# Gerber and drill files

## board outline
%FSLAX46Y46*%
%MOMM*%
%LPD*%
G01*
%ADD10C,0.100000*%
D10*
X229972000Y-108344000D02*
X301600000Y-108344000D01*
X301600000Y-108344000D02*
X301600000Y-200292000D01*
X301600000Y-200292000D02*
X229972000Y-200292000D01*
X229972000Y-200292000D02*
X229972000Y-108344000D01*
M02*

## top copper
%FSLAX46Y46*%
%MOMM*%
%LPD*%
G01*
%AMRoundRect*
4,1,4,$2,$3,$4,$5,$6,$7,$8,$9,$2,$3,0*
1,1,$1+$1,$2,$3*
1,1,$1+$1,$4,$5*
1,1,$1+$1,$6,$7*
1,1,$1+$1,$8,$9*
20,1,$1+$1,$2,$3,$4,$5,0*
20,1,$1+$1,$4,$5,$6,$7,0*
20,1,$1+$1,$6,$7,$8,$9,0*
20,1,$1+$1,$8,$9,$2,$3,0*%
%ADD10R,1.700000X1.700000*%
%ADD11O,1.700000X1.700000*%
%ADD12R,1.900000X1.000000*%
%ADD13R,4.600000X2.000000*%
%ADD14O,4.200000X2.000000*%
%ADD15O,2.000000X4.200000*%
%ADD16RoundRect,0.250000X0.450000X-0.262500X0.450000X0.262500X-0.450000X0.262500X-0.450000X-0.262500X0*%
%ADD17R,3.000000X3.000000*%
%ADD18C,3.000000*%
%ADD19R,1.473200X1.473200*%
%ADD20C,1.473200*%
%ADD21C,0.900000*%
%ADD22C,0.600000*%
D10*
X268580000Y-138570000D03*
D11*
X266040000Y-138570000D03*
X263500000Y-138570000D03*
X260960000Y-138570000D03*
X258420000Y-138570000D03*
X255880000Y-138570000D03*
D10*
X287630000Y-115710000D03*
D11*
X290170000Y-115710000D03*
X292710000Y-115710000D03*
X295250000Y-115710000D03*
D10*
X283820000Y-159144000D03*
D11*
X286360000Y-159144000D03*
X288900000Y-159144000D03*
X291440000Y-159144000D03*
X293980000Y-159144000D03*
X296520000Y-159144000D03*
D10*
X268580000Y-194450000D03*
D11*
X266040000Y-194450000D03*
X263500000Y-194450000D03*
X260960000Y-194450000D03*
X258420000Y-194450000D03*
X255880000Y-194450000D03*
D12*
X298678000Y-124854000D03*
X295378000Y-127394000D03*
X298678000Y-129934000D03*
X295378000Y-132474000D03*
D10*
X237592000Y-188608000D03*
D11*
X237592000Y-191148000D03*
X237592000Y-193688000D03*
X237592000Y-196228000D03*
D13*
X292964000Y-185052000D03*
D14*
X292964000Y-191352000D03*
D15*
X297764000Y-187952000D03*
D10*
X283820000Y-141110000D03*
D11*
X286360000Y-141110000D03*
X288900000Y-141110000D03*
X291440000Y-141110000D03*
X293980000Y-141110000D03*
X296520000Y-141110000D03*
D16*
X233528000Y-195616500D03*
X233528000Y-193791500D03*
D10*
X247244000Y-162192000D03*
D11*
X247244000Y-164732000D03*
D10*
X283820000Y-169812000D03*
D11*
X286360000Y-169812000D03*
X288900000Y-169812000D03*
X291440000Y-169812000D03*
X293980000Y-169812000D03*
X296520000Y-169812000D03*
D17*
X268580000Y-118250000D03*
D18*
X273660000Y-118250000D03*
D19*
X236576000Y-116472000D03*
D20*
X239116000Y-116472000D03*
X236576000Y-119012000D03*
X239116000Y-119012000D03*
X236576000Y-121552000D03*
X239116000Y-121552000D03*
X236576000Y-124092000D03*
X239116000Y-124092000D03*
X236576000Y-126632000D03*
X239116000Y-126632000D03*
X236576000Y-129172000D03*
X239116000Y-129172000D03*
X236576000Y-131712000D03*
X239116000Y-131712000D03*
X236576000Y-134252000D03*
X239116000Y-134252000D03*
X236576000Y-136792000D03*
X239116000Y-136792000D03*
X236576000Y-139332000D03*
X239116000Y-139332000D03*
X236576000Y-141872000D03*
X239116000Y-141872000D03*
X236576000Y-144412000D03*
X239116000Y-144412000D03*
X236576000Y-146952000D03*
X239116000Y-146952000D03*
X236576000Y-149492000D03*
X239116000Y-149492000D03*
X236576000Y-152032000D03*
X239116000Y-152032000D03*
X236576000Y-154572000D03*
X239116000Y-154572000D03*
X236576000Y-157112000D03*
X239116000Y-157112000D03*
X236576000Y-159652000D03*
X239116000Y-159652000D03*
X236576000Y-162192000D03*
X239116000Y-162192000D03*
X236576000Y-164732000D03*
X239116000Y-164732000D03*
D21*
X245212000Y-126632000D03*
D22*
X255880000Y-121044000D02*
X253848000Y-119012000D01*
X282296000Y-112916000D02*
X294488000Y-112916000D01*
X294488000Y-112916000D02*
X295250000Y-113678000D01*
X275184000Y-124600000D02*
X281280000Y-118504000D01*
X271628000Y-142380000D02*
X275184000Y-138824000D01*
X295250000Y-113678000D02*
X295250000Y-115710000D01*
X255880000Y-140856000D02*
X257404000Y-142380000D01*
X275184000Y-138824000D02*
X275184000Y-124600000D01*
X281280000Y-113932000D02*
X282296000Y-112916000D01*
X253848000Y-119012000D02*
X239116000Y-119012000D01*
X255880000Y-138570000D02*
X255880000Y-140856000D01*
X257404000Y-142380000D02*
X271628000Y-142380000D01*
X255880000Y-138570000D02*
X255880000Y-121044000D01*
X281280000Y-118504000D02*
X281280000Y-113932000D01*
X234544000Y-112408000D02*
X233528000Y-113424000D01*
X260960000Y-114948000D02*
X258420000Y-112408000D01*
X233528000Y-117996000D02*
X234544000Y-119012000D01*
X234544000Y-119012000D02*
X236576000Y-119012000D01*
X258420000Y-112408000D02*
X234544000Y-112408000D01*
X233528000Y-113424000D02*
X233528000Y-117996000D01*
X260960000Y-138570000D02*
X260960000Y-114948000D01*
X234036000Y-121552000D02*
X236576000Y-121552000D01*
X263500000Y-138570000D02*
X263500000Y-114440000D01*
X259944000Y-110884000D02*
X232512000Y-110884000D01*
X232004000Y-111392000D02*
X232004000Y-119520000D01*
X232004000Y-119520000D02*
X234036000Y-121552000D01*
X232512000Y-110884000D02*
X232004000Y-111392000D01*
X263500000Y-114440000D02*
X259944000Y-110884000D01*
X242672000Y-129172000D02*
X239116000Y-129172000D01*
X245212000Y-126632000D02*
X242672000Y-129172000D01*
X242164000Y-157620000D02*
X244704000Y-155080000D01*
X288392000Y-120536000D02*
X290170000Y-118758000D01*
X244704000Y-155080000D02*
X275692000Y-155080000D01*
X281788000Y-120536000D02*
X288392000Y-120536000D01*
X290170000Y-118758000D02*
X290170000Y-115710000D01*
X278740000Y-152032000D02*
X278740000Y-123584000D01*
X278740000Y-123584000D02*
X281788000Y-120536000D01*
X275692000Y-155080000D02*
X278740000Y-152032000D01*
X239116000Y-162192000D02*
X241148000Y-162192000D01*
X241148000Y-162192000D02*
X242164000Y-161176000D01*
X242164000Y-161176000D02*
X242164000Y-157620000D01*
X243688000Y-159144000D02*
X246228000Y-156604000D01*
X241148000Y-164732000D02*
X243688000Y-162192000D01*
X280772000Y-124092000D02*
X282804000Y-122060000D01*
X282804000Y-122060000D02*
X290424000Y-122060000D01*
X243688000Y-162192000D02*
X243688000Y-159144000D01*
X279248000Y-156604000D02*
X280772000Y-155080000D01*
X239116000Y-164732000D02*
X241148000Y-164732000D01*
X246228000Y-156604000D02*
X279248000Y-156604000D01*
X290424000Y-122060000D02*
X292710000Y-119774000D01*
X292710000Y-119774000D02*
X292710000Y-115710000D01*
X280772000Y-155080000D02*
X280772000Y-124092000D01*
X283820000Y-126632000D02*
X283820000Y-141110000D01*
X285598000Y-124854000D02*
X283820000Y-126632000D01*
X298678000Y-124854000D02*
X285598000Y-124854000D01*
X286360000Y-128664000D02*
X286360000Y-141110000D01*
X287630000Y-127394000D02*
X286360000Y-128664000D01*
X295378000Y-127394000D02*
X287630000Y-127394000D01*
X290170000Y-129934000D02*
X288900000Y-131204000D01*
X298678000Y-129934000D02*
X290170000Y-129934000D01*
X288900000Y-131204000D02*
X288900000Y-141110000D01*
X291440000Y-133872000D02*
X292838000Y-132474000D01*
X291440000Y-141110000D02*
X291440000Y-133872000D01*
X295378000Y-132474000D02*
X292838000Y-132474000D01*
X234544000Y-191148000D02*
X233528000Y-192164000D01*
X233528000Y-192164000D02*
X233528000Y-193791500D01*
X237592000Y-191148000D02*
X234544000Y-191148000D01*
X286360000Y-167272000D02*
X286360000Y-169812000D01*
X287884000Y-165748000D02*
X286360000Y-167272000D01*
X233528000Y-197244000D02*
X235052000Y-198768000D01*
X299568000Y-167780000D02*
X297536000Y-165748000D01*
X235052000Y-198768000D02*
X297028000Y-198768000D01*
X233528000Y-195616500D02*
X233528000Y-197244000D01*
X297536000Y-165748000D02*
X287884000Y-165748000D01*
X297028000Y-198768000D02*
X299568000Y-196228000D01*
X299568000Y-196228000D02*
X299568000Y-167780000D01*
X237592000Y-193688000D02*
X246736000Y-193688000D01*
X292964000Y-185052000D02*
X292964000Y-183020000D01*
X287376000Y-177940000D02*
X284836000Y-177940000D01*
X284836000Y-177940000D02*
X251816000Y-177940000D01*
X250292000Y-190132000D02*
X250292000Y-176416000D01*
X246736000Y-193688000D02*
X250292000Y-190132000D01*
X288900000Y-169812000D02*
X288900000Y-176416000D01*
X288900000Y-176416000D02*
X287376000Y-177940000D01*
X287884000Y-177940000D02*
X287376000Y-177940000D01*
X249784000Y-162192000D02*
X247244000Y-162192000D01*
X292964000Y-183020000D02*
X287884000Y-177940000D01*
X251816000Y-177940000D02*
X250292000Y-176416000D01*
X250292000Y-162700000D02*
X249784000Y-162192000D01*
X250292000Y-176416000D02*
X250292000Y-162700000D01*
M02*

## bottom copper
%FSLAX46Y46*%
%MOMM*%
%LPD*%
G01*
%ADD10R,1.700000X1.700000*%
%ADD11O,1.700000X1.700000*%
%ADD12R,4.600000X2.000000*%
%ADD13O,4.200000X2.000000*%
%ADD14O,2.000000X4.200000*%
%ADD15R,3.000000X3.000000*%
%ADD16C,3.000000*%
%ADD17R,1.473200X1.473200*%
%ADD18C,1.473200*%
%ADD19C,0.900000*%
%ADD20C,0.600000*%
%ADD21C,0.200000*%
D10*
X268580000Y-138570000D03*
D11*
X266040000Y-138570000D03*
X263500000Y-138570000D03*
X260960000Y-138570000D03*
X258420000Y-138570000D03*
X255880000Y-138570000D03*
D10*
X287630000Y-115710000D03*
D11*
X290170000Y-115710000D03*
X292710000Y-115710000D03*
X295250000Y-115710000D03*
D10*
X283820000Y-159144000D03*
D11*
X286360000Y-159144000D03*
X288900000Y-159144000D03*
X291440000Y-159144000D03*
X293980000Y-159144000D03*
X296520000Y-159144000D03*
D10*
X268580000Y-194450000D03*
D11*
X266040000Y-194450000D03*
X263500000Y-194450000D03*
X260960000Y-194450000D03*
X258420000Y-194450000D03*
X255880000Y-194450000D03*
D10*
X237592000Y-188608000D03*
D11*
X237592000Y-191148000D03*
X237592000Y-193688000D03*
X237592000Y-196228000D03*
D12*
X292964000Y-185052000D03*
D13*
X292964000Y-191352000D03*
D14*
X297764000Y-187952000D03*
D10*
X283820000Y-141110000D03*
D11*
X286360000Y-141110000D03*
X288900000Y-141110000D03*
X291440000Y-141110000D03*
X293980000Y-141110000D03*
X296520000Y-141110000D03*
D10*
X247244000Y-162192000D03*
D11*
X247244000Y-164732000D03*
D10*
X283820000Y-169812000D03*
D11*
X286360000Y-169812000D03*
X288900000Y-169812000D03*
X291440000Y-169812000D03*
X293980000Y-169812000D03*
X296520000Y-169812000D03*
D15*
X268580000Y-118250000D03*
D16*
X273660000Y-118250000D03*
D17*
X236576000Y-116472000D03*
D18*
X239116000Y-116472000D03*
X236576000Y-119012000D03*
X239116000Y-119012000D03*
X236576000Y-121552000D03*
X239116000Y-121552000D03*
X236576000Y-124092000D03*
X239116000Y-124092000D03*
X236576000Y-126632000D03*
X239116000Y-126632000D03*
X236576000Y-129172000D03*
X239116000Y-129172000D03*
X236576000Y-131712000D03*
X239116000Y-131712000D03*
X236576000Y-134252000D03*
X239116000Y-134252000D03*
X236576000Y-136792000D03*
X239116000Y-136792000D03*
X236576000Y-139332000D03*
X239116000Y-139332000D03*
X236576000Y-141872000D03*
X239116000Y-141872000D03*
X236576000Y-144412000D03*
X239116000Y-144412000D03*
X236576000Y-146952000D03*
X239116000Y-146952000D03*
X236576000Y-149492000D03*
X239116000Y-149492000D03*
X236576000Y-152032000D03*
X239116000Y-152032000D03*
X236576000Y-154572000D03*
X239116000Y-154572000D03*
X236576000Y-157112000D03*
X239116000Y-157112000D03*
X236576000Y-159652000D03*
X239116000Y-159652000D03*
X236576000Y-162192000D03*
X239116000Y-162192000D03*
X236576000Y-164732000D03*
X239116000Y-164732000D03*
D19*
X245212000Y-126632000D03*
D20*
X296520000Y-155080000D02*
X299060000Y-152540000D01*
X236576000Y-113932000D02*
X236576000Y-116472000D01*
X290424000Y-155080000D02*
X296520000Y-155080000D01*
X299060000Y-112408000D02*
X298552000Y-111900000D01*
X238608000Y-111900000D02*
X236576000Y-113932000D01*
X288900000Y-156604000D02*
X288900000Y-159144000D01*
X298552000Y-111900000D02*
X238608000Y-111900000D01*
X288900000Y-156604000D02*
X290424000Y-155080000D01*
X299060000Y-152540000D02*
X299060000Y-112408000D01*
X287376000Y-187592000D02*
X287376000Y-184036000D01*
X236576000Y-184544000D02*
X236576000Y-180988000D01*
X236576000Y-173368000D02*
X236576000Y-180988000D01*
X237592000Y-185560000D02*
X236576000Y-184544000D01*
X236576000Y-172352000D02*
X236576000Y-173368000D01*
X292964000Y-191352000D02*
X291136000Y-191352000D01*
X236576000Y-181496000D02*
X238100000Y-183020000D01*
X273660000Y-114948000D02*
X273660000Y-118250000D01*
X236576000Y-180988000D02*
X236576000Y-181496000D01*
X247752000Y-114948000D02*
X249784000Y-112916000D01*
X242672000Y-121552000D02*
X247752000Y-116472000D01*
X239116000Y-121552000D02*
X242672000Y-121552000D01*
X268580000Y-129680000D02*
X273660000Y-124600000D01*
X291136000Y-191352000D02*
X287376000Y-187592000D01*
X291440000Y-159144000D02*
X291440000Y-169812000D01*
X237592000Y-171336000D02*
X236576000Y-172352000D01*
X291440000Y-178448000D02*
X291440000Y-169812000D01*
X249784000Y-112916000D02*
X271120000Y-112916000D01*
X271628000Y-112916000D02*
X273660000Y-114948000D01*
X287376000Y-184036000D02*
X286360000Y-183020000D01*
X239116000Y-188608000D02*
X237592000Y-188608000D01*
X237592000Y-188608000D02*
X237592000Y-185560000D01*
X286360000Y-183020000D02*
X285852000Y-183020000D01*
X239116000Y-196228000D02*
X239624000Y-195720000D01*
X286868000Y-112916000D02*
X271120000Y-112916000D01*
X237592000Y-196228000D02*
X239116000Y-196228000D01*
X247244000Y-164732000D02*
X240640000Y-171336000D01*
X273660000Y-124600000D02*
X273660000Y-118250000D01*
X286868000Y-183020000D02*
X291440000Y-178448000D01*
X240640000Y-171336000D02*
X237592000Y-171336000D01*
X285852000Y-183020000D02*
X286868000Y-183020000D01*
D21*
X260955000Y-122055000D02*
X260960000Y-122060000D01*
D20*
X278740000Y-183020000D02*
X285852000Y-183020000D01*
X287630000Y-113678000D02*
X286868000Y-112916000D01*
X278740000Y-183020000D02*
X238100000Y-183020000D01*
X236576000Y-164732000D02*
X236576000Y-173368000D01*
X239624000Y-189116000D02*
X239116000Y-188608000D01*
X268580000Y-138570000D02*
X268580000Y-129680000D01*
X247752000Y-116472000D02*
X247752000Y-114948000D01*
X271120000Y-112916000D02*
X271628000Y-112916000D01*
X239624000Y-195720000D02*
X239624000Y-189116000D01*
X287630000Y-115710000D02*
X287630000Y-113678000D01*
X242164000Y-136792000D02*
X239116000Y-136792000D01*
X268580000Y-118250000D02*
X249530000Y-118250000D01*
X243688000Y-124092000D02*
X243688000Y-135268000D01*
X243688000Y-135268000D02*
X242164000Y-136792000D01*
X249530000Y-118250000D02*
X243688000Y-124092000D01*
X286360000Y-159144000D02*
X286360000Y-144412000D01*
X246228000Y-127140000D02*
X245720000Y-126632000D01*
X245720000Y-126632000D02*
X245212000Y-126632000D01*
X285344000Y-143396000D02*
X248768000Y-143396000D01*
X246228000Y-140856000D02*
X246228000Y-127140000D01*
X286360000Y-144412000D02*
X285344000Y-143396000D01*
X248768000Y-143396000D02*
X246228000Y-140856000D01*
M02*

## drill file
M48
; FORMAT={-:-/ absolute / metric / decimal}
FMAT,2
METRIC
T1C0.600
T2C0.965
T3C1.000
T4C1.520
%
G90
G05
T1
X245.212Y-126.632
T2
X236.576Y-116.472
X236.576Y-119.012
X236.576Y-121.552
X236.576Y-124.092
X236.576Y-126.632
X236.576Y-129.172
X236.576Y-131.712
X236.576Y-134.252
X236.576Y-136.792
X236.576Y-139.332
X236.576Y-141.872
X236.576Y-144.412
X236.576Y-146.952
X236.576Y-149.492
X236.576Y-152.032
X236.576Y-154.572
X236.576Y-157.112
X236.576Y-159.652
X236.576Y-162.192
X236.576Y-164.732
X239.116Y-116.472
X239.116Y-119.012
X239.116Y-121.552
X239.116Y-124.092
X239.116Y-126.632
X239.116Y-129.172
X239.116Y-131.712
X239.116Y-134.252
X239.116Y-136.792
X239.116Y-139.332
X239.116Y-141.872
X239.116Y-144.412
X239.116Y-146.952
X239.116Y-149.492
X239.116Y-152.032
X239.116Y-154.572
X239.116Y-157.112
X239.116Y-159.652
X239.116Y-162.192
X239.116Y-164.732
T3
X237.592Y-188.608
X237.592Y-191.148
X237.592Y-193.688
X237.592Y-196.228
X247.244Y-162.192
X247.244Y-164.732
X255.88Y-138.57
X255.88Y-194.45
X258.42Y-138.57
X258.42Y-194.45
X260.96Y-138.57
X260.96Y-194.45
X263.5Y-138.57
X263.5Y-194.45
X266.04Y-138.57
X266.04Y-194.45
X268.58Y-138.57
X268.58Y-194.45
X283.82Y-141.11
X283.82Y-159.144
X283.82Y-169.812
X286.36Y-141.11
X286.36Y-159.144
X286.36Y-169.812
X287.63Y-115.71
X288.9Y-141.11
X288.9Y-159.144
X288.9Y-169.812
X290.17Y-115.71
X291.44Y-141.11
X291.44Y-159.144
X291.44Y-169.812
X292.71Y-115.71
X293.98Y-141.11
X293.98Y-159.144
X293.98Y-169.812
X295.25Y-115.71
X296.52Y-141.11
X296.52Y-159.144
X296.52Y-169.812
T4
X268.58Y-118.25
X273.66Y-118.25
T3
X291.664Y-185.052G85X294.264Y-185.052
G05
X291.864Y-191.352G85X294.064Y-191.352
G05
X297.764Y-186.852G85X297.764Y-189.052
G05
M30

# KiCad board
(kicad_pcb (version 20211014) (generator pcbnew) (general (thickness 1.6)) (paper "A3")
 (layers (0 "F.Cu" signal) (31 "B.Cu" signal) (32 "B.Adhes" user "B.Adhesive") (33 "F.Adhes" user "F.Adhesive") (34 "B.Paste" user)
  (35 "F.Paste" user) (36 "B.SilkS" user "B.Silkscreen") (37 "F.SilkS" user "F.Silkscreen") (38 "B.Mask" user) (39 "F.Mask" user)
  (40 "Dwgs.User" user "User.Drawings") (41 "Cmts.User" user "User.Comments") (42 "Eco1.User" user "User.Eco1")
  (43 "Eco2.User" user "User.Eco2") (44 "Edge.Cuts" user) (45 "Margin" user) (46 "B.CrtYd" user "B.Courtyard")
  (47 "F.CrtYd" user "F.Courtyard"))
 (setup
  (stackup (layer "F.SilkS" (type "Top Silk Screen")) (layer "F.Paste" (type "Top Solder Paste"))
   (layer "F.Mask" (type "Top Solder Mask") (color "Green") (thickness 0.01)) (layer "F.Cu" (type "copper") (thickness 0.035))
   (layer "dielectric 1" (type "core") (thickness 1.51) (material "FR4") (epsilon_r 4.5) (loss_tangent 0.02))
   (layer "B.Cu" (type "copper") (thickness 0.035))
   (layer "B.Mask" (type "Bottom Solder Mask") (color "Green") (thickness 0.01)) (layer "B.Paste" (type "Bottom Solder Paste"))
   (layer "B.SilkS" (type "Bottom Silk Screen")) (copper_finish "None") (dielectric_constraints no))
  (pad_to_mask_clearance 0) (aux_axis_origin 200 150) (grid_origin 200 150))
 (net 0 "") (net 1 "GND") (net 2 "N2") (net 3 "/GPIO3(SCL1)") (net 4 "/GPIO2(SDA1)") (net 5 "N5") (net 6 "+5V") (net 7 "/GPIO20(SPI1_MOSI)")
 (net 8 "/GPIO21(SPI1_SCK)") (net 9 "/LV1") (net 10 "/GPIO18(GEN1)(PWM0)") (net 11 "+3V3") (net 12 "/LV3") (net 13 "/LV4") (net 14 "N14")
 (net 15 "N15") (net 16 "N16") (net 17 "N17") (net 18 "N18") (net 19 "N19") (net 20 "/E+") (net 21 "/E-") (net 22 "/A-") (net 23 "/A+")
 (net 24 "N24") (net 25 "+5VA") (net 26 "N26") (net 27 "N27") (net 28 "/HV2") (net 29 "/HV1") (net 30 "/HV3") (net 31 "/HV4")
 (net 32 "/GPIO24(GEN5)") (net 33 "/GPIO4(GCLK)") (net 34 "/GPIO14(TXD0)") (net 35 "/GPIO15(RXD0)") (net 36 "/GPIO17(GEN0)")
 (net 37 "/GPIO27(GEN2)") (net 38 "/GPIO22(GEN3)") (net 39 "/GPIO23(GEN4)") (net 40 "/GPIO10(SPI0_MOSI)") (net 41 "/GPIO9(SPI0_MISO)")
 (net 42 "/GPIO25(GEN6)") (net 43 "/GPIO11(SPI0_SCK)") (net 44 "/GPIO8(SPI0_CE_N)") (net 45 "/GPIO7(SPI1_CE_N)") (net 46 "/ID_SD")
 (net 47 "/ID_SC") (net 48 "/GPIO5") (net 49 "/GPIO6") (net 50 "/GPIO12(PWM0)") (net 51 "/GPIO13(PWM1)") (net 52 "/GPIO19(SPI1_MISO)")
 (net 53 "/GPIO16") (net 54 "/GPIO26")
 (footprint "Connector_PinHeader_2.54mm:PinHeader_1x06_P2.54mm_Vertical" (layer "F.Cu") (at 268.58 138.57 -90)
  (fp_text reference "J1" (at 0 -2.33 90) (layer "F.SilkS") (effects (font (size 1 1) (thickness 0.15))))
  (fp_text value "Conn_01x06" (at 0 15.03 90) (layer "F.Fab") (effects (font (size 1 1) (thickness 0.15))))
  (pad "1" thru_hole rect (at 0 0 270) (size 1.7 1.7) (drill 1) (layers *.Cu *.Mask) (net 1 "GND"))
  (pad "2" thru_hole oval (at 0 2.54 270) (size 1.7 1.7) (drill 1) (layers *.Cu *.Mask) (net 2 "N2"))
  (pad "3" thru_hole oval (at 0 5.08 270) (size 1.7 1.7) (drill 1) (layers *.Cu *.Mask) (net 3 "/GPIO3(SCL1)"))
  (pad "4" thru_hole oval (at 0 7.62 270) (size 1.7 1.7) (drill 1) (layers *.Cu *.Mask) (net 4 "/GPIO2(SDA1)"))
  (pad "5" thru_hole oval (at 0 10.16 270) (size 1.7 1.7) (drill 1) (layers *.Cu *.Mask) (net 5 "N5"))
  (pad "6" thru_hole oval (at 0 12.7 270) (size 1.7 1.7) (drill 1) (layers *.Cu *.Mask) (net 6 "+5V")))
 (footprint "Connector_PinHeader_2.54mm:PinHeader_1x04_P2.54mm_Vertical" (layer "F.Cu") (at 287.63 115.71 90)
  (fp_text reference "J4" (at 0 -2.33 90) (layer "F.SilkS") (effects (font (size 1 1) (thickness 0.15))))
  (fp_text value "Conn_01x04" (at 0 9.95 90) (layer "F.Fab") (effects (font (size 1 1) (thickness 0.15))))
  (pad "1" thru_hole rect (at 0 0 90) (size 1.7 1.7) (drill 1) (layers *.Cu *.Mask) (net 1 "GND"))
  (pad "2" thru_hole oval (at 0 2.54 90) (size 1.7 1.7) (drill 1) (layers *.Cu *.Mask) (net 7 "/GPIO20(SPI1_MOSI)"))
  (pad "3" thru_hole oval (at 0 5.08 90) (size 1.7 1.7) (drill 1) (layers *.Cu *.Mask) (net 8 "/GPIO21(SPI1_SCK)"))
  (pad "4" thru_hole oval (at 0 7.62 90) (size 1.7 1.7) (drill 1) (layers *.Cu *.Mask) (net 6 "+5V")))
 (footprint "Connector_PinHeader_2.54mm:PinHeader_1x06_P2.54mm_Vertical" (layer "F.Cu") (at 283.82 159.144 90)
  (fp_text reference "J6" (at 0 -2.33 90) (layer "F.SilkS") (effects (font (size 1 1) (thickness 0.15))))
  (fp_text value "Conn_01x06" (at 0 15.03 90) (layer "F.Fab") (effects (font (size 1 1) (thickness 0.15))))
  (pad "1" thru_hole rect (at 0 0 90) (size 1.7 1.7) (drill 1) (layers *.Cu *.Mask) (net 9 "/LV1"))
  (pad "2" thru_hole oval (at 0 2.54 90) (size 1.7 1.7) (drill 1) (layers *.Cu *.Mask) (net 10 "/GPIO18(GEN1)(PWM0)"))
  (pad "3" thru_hole oval (at 0 5.08 90) (size 1.7 1.7) (drill 1) (layers *.Cu *.Mask) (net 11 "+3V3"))
  (pad "4" thru_hole oval (at 0 7.62 90) (size 1.7 1.7) (drill 1) (layers *.Cu *.Mask) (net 1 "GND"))
  (pad "5" thru_hole oval (at 0 10.16 90) (size 1.7 1.7) (drill 1) (layers *.Cu *.Mask) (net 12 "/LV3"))
  (pad "6" thru_hole oval (at 0 12.7 90) (size 1.7 1.7) (drill 1) (layers *.Cu *.Mask) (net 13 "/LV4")))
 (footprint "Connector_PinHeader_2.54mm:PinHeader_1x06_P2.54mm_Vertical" (layer "F.Cu") (at 268.58 194.45 -90)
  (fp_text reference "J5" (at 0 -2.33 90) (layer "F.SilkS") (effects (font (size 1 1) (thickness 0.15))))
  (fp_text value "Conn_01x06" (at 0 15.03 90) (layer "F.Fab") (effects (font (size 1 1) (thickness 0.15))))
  (pad "1" thru_hole rect (at 0 0 270) (size 1.7 1.7) (drill 1) (layers *.Cu *.Mask) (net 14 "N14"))
  (pad "2" thru_hole oval (at 0 2.54 270) (size 1.7 1.7) (drill 1) (layers *.Cu *.Mask) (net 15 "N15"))
  (pad "3" thru_hole oval (at 0 5.08 270) (size 1.7 1.7) (drill 1) (layers *.Cu *.Mask) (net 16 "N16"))
  (pad "4" thru_hole oval (at 0 7.62 270) (size 1.7 1.7) (drill 1) (layers *.Cu *.Mask) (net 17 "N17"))
  (pad "5" thru_hole oval (at 0 10.16 270) (size 1.7 1.7) (drill 1) (layers *.Cu *.Mask) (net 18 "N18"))
  (pad "6" thru_hole oval (at 0 12.7 270) (size 1.7 1.7) (drill 1) (layers *.Cu *.Mask) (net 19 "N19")))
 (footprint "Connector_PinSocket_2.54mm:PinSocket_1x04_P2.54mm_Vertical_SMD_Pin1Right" (layer "F.Cu") (at 297.028 128.664)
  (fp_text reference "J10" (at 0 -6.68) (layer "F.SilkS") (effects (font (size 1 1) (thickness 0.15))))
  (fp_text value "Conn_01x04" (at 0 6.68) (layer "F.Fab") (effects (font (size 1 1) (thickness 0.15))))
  (pad "1" smd rect (at 1.65 -3.81) (size 1.9 1) (layers "F.Cu" "F.Paste" "F.Mask") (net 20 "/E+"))
  (pad "2" smd rect (at -1.65 -1.27) (size 1.9 1) (layers "F.Cu" "F.Paste" "F.Mask") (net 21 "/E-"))
  (pad "3" smd rect (at 1.65 1.27) (size 1.9 1) (layers "F.Cu" "F.Paste" "F.Mask") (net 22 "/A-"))
  (pad "4" smd rect (at -1.65 3.81) (size 1.9 1) (layers "F.Cu" "F.Paste" "F.Mask") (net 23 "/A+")))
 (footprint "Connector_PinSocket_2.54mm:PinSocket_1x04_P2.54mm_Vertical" (layer "F.Cu") (at 237.592 188.608)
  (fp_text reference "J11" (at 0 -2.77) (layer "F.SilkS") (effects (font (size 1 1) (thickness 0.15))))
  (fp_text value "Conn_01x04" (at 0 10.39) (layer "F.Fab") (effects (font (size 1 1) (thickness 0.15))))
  (pad "1" thru_hole rect (at 0 0) (size 1.7 1.7) (drill 1) (layers *.Cu *.Mask) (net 1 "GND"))
  (pad "2" thru_hole oval (at 0 2.54) (size 1.7 1.7) (drill 1) (layers *.Cu *.Mask) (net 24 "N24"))
  (pad "3" thru_hole oval (at 0 5.08) (size 1.7 1.7) (drill 1) (layers *.Cu *.Mask) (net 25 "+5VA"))
  (pad "4" thru_hole oval (at 0 7.62) (size 1.7 1.7) (drill 1) (layers *.Cu *.Mask) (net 1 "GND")))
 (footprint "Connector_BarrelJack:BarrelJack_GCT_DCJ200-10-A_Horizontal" (layer "F.Cu") (at 292.964 185.052)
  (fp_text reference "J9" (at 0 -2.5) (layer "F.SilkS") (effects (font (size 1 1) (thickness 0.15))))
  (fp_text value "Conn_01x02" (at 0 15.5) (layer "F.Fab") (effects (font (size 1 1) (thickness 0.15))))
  (pad "1" thru_hole rect (at 0 0) (size 4.6 2) (drill oval 3.6 1) (layers *.Cu *.Mask) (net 25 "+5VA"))
  (pad "2" thru_hole oval (at 0 6.3) (size 4.2 2) (drill oval 3.2 1) (layers *.Cu *.Mask) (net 1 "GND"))
  (pad "3" thru_hole oval (at 4.8 2.9) (size 2 4.2) (drill oval 1 3.2) (layers *.Cu *.Mask)))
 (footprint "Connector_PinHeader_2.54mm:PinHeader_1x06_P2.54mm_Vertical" (layer "F.Cu") (at 283.82 141.11 90)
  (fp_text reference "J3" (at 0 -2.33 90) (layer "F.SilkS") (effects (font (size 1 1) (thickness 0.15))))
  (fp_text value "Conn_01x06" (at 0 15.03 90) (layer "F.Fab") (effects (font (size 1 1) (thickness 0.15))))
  (pad "1" thru_hole rect (at 0 0 90) (size 1.7 1.7) (drill 1) (layers *.Cu *.Mask) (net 20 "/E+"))
  (pad "2" thru_hole oval (at 0 2.54 90) (size 1.7 1.7) (drill 1) (layers *.Cu *.Mask) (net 21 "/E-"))
  (pad "3" thru_hole oval (at 0 5.08 90) (size 1.7 1.7) (drill 1) (layers *.Cu *.Mask) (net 22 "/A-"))
  (pad "4" thru_hole oval (at 0 7.62 90) (size 1.7 1.7) (drill 1) (layers *.Cu *.Mask) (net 23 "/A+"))
  (pad "5" thru_hole oval (at 0 10.16 90) (size 1.7 1.7) (drill 1) (layers *.Cu *.Mask) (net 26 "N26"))
  (pad "6" thru_hole oval (at 0 12.7 90) (size 1.7 1.7) (drill 1) (layers *.Cu *.Mask) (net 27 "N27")))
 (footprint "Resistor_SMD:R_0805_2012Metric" (layer "F.Cu") (at 233.528 194.704 90)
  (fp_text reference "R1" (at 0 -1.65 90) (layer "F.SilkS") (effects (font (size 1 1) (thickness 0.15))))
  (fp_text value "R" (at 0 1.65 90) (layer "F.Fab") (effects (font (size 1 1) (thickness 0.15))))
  (pad "1" smd roundrect (at -0.9125 0 90) (size 1.025 1.4) (layers "F.Cu" "F.Paste" "F.Mask") (roundrect_rratio 0.243902) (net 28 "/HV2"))
  (pad "2" smd roundrect (at 0.9125 0 90) (size 1.025 1.4) (layers "F.Cu" "F.Paste" "F.Mask") (roundrect_rratio 0.243902) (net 24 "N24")))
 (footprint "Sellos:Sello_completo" (layer "F.Cu") (at 265.532 148.984)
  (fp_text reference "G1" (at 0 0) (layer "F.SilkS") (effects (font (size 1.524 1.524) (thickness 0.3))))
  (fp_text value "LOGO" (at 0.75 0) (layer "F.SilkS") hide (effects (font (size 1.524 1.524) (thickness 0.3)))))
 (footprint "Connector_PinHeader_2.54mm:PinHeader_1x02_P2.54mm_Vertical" (layer "F.Cu") (at 247.244 162.192)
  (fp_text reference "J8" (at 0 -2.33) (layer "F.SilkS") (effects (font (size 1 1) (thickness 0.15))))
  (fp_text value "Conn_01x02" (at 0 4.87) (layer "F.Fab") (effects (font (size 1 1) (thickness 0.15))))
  (pad "1" thru_hole rect (at 0 0) (size 1.7 1.7) (drill 1) (layers *.Cu *.Mask) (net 25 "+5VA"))
  (pad "2" thru_hole oval (at 0 2.54) (size 1.7 1.7) (drill 1) (layers *.Cu *.Mask) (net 1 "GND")))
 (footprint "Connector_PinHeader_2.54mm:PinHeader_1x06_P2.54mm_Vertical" (layer "F.Cu") (at 283.82 169.812 90)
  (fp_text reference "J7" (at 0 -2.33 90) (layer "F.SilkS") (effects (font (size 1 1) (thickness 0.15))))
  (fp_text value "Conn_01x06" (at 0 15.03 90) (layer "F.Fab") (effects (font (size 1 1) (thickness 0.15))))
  (pad "1" thru_hole rect (at 0 0 90) (size 1.7 1.7) (drill 1) (layers *.Cu *.Mask) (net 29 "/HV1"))
  (pad "2" thru_hole oval (at 0 2.54 90) (size 1.7 1.7) (drill 1) (layers *.Cu *.Mask) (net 28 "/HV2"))
  (pad "3" thru_hole oval (at 0 5.08 90) (size 1.7 1.7) (drill 1) (layers *.Cu *.Mask) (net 25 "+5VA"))
  (pad "4" thru_hole oval (at 0 7.62 90) (size 1.7 1.7) (drill 1) (layers *.Cu *.Mask) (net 1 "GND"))
  (pad "5" thru_hole oval (at 0 10.16 90) (size 1.7 1.7) (drill 1) (layers *.Cu *.Mask) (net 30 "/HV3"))
  (pad "6" thru_hole oval (at 0 12.7 90) (size 1.7 1.7) (drill 1) (layers *.Cu *.Mask) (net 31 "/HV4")))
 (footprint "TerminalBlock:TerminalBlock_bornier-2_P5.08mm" (layer "F.Cu") (at 268.58 118.25)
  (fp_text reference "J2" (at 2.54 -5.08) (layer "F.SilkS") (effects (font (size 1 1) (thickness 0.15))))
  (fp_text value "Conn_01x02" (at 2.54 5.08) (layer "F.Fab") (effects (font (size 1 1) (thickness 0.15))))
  (pad "1" thru_hole rect (at 0 0) (size 3 3) (drill 1.52) (layers *.Cu *.Mask) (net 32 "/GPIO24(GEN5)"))
  (pad "2" thru_hole circle (at 5.08 0) (size 3 3) (drill 1.52) (layers *.Cu *.Mask) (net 1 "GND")))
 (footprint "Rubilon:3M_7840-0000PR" (layer "F.Cu") (at 239.116 116.472 90)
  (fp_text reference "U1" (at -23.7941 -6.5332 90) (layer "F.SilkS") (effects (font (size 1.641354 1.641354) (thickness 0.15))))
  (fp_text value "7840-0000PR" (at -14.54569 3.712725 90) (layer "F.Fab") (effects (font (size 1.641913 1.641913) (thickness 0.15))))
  (pad "1" thru_hole rect locked (at 0 -2.54 90) (size 1.4732 1.4732) (drill 0.9652) (layers *.Cu *.Mask) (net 11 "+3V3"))
  (pad "2" thru_hole circle locked (at 0 0 90) (size 1.4732 1.4732) (drill 0.9652) (layers *.Cu *.Mask) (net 6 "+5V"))
  (pad "3" thru_hole circle locked (at -2.54 -2.54 90) (size 1.4732 1.4732) (drill 0.9652) (layers *.Cu *.Mask) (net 4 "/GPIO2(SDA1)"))
  (pad "4" thru_hole circle locked (at -2.54 0 90) (size 1.4732 1.4732) (drill 0.9652) (layers *.Cu *.Mask) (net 6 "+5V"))
  (pad "5" thru_hole circle locked (at -5.08 -2.54 90) (size 1.4732 1.4732) (drill 0.9652) (layers *.Cu *.Mask) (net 3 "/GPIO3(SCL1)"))
  (pad "6" thru_hole circle locked (at -5.08 0 90) (size 1.4732 1.4732) (drill 0.9652) (layers *.Cu *.Mask) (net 1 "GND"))
  (pad "7" thru_hole circle locked (at -7.62 -2.54 90) (size 1.4732 1.4732) (drill 0.9652) (layers *.Cu *.Mask) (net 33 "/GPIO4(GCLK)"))
  (pad "8" thru_hole circle locked (at -7.62 0 90) (size 1.4732 1.4732) (drill 0.9652) (layers *.Cu *.Mask) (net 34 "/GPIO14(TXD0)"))
  (pad "9" thru_hole circle locked (at -10.16 -2.54 90) (size 1.4732 1.4732) (drill 0.9652) (layers *.Cu *.Mask) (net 1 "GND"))
  (pad "10" thru_hole circle locked (at -10.16 0 90) (size 1.4732 1.4732) (drill 0.9652) (layers *.Cu *.Mask) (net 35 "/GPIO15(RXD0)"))
  (pad "11" thru_hole circle locked (at -12.7 -2.54 90) (size 1.4732 1.4732) (drill 0.9652) (layers *.Cu *.Mask) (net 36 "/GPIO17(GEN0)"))
  (pad "12" thru_hole circle locked (at -12.7 0 90) (size 1.4732 1.4732) (drill 0.9652) (layers *.Cu *.Mask) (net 10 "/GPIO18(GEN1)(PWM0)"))
  (pad "13" thru_hole circle locked (at -15.24 -2.54 90) (size 1.4732 1.4732) (drill 0.9652) (layers *.Cu *.Mask) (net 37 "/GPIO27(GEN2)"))
  (pad "14" thru_hole circle locked (at -15.24 0 90) (size 1.4732 1.4732) (drill 0.9652) (layers *.Cu *.Mask) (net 1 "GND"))
  (pad "15" thru_hole circle locked (at -17.78 -2.54 90) (size 1.4732 1.4732) (drill 0.9652) (layers *.Cu *.Mask) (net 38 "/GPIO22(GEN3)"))
  (pad "16" thru_hole circle locked (at -17.78 0 90) (size 1.4732 1.4732) (drill 0.9652) (layers *.Cu *.Mask) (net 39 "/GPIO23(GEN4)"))
  (pad "17" thru_hole circle locked (at -20.32 -2.54 90) (size 1.4732 1.4732) (drill 0.9652) (layers *.Cu *.Mask) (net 11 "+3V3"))
  (pad "18" thru_hole circle locked (at -20.32 0 90) (size 1.4732 1.4732) (drill 0.9652) (layers *.Cu *.Mask) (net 32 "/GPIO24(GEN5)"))
  (pad "19" thru_hole circle locked (at -22.86 -2.54 90) (size 1.4732 1.4732) (drill 0.9652) (layers *.Cu *.Mask)
   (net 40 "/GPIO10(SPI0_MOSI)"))
  (pad "20" thru_hole circle locked (at -22.86 0 90) (size 1.4732 1.4732) (drill 0.9652) (layers *.Cu *.Mask) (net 1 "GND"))
  (pad "21" thru_hole circle locked (at -25.4 -2.54 90) (size 1.4732 1.4732) (drill 0.9652) (layers *.Cu *.Mask)
   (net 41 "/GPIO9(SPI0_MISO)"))
  (pad "22" thru_hole circle locked (at -25.4 0 90) (size 1.4732 1.4732) (drill 0.9652) (layers *.Cu *.Mask) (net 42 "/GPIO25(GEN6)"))
  (pad "23" thru_hole circle locked (at -27.94 -2.54 90) (size 1.4732 1.4732) (drill 0.9652) (layers *.Cu *.Mask)
   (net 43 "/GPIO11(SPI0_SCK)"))
  (pad "24" thru_hole circle locked (at -27.94 0 90) (size 1.4732 1.4732) (drill 0.9652) (layers *.Cu *.Mask) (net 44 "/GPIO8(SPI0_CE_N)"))
  (pad "25" thru_hole circle locked (at -30.48 -2.54 90) (size 1.4732 1.4732) (drill 0.9652) (layers *.Cu *.Mask) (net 1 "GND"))
  (pad "26" thru_hole circle locked (at -30.48 0 90) (size 1.4732 1.4732) (drill 0.9652) (layers *.Cu *.Mask) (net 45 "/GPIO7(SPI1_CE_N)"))
  (pad "27" thru_hole circle locked (at -33.02 -2.54 90) (size 1.4732 1.4732) (drill 0.9652) (layers *.Cu *.Mask) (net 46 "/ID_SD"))
  (pad "28" thru_hole circle locked (at -33.02 0 90) (size 1.4732 1.4732) (drill 0.9652) (layers *.Cu *.Mask) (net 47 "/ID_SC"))
  (pad "29" thru_hole circle locked (at -35.56 -2.54 90) (size 1.4732 1.4732) (drill 0.9652) (layers *.Cu *.Mask) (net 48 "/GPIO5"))
  (pad "30" thru_hole circle locked (at -35.56 0 90) (size 1.4732 1.4732) (drill 0.9652) (layers *.Cu *.Mask) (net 1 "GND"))
  (pad "31" thru_hole circle locked (at -38.1 -2.54 90) (size 1.4732 1.4732) (drill 0.9652) (layers *.Cu *.Mask) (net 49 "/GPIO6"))
  (pad "32" thru_hole circle locked (at -38.1 0 90) (size 1.4732 1.4732) (drill 0.9652) (layers *.Cu *.Mask) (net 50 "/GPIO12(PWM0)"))
  (pad "33" thru_hole circle locked (at -40.64 -2.54 90) (size 1.4732 1.4732) (drill 0.9652) (layers *.Cu *.Mask) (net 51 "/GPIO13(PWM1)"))
  (pad "34" thru_hole circle locked (at -40.64 0 90) (size 1.4732 1.4732) (drill 0.9652) (layers *.Cu *.Mask) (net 1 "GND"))
  (pad "35" thru_hole circle locked (at -43.18 -2.54 90) (size 1.4732 1.4732) (drill 0.9652) (layers *.Cu *.Mask)
   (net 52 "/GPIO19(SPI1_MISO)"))
  (pad "36" thru_hole circle locked (at -43.18 0 90) (size 1.4732 1.4732) (drill 0.9652) (layers *.Cu *.Mask) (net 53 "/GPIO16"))
  (pad "37" thru_hole circle locked (at -45.72 -2.54 90) (size 1.4732 1.4732) (drill 0.9652) (layers *.Cu *.Mask) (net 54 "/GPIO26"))
  (pad "38" thru_hole circle locked (at -45.72 0 90) (size 1.4732 1.4732) (drill 0.9652) (layers *.Cu *.Mask) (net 7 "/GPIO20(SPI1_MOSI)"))
  (pad "39" thru_hole circle locked (at -48.26 -2.54 90) (size 1.4732 1.4732) (drill 0.9652) (layers *.Cu *.Mask) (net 1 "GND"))
  (pad "40" thru_hole circle locked (at -48.26 0 90) (size 1.4732 1.4732) (drill 0.9652) (layers *.Cu *.Mask) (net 8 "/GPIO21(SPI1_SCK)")))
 (gr_line (start 229.972 108.344) (end 301.6 108.344) (layer "Edge.Cuts") (width 0.1))
 (gr_line (start 301.6 108.344) (end 301.6 200.292) (layer "Edge.Cuts") (width 0.1))
 (gr_line (start 301.6 200.292) (end 229.972 200.292) (layer "Edge.Cuts") (width 0.1))
 (gr_line (start 229.972 200.292) (end 229.972 108.344) (layer "Edge.Cuts") (width 0.1))
 (segment (start 296.52 155.08) (end 299.06 152.54) (width 0.6) (layer "B.Cu") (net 11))
 (segment (start 236.576 113.932) (end 236.576 116.472) (width 0.6) (layer "B.Cu") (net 11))
 (segment (start 290.424 155.08) (end 296.52 155.08) (width 0.6) (layer "B.Cu") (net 11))
 (segment (start 299.06 112.408) (end 298.552 111.9) (width 0.6) (layer "B.Cu") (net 11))
 (segment (start 238.608 111.9) (end 236.576 113.932) (width 0.6) (layer "B.Cu") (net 11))
 (segment (start 288.9 156.604) (end 288.9 159.144) (width 0.6) (layer "B.Cu") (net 11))
 (segment (start 298.552 111.9) (end 238.608 111.9) (width 0.6) (layer "B.Cu") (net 11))
 (segment (start 288.9 156.604) (end 290.424 155.08) (width 0.6) (layer "B.Cu") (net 11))
 (segment (start 299.06 152.54) (end 299.06 112.408) (width 0.6) (layer "B.Cu") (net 11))
 (segment (start 255.88 121.044) (end 253.848 119.012) (width 0.6) (layer "F.Cu") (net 6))
 (segment (start 282.296 112.916) (end 294.488 112.916) (width 0.6) (layer "F.Cu") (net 6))
 (segment (start 294.488 112.916) (end 295.25 113.678) (width 0.6) (layer "F.Cu") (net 6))
 (segment (start 275.184 124.6) (end 281.28 118.504) (width 0.6) (layer "F.Cu") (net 6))
 (segment (start 271.628 142.38) (end 275.184 138.824) (width 0.6) (layer "F.Cu") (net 6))
 (segment (start 295.25 113.678) (end 295.25 115.71) (width 0.6) (layer "F.Cu") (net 6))
 (segment (start 255.88 140.856) (end 257.404 142.38) (width 0.6) (layer "F.Cu") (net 6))
 (segment (start 275.184 138.824) (end 275.184 124.6) (width 0.6) (layer "F.Cu") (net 6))
 (segment (start 281.28 113.932) (end 282.296 112.916) (width 0.6) (layer "F.Cu") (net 6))
 (segment (start 253.848 119.012) (end 239.116 119.012) (width 0.6) (layer "F.Cu") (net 6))
 (segment (start 255.88 138.57) (end 255.88 140.856) (width 0.6) (layer "F.Cu") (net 6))
 (segment (start 257.404 142.38) (end 271.628 142.38) (width 0.6) (layer "F.Cu") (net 6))
 (segment (start 255.88 138.57) (end 255.88 121.044) (width 0.6) (layer "F.Cu") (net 6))
 (segment (start 281.28 118.504) (end 281.28 113.932) (width 0.6) (layer "F.Cu") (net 6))
 (segment (start 287.376 187.592) (end 287.376 184.036) (width 0.6) (layer "B.Cu") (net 1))
 (segment (start 236.576 184.544) (end 236.576 180.988) (width 0.6) (layer "B.Cu") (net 1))
 (segment (start 236.576 173.368) (end 236.576 180.988) (width 0.6) (layer "B.Cu") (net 1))
 (segment (start 237.592 185.56) (end 236.576 184.544) (width 0.6) (layer "B.Cu") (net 1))
 (segment (start 236.576 172.352) (end 236.576 173.368) (width 0.6) (layer "B.Cu") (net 1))
 (segment (start 292.964 191.352) (end 291.136 191.352) (width 0.6) (layer "B.Cu") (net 1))
 (segment (start 236.576 181.496) (end 238.1 183.02) (width 0.6) (layer "B.Cu") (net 1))
 (segment (start 273.66 114.948) (end 273.66 118.25) (width 0.6) (layer "B.Cu") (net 1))
 (segment (start 236.576 180.988) (end 236.576 181.496) (width 0.6) (layer "B.Cu") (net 1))
 (segment (start 247.752 114.948) (end 249.784 112.916) (width 0.6) (layer "B.Cu") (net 1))
 (segment (start 242.672 121.552) (end 247.752 116.472) (width 0.6) (layer "B.Cu") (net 1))
 (segment (start 239.116 121.552) (end 242.672 121.552) (width 0.6) (layer "B.Cu") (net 1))
 (segment (start 268.58 129.68) (end 273.66 124.6) (width 0.6) (layer "B.Cu") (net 1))
 (segment (start 291.136 191.352) (end 287.376 187.592) (width 0.6) (layer "B.Cu") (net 1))
 (segment (start 291.44 159.144) (end 291.44 169.812) (width 0.6) (layer "B.Cu") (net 1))
 (segment (start 237.592 171.336) (end 236.576 172.352) (width 0.6) (layer "B.Cu") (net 1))
 (segment (start 291.44 178.448) (end 291.44 169.812) (width 0.6) (layer "B.Cu") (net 1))
 (segment (start 249.784 112.916) (end 271.12 112.916) (width 0.6) (layer "B.Cu") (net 1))
 (segment (start 271.628 112.916) (end 273.66 114.948) (width 0.6) (layer "B.Cu") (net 1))
 (segment (start 287.376 184.036) (end 286.36 183.02) (width 0.6) (layer "B.Cu") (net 1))
 (segment (start 239.116 188.608) (end 237.592 188.608) (width 0.6) (layer "B.Cu") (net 1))
 (segment (start 237.592 188.608) (end 237.592 185.56) (width 0.6) (layer "B.Cu") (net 1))
 (segment (start 286.36 183.02) (end 285.852 183.02) (width 0.6) (layer "B.Cu") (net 1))
 (segment (start 239.116 196.228) (end 239.624 195.72) (width 0.6) (layer "B.Cu") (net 1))
 (segment (start 286.868 112.916) (end 271.12 112.916) (width 0.6) (layer "B.Cu") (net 1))
 (segment (start 237.592 196.228) (end 239.116 196.228) (width 0.6) (layer "B.Cu") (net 1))
 (segment (start 247.244 164.732) (end 240.64 171.336) (width 0.6) (layer "B.Cu") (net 1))
 (segment (start 273.66 124.6) (end 273.66 118.25) (width 0.6) (layer "B.Cu") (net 1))
 (segment (start 286.868 183.02) (end 291.44 178.448) (width 0.6) (layer "B.Cu") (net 1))
 (segment (start 240.64 171.336) (end 237.592 171.336) (width 0.6) (layer "B.Cu") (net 1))
 (segment (start 285.852 183.02) (end 286.868 183.02) (width 0.6) (layer "B.Cu") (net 1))
 (segment (start 260.955 122.055) (end 260.96 122.06) (width 0.2) (layer "B.Cu") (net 1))
 (segment (start 278.74 183.02) (end 285.852 183.02) (width 0.6) (layer "B.Cu") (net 1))
 (segment (start 287.63 113.678) (end 286.868 112.916) (width 0.6) (layer "B.Cu") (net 1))
 (segment (start 278.74 183.02) (end 238.1 183.02) (width 0.6) (layer "B.Cu") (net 1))
 (segment (start 236.576 164.732) (end 236.576 173.368) (width 0.6) (layer "B.Cu") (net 1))
 (segment (start 239.624 189.116) (end 239.116 188.608) (width 0.6) (layer "B.Cu") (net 1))
 (segment (start 268.58 138.57) (end 268.58 129.68) (width 0.6) (layer "B.Cu") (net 1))
 (segment (start 247.752 116.472) (end 247.752 114.948) (width 0.6) (layer "B.Cu") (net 1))
 (segment (start 271.12 112.916) (end 271.628 112.916) (width 0.6) (layer "B.Cu") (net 1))
 (segment (start 239.624 195.72) (end 239.624 189.116) (width 0.6) (layer "B.Cu") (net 1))
 (segment (start 287.63 115.71) (end 287.63 113.678) (width 0.6) (layer "B.Cu") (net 1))
 (segment (start 234.544 112.408) (end 233.528 113.424) (width 0.6) (layer "F.Cu") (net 4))
 (segment (start 260.96 114.948) (end 258.42 112.408) (width 0.6) (layer "F.Cu") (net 4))
 (segment (start 233.528 117.996) (end 234.544 119.012) (width 0.6) (layer "F.Cu") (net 4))
 (segment (start 234.544 119.012) (end 236.576 119.012) (width 0.6) (layer "F.Cu") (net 4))
 (segment (start 258.42 112.408) (end 234.544 112.408) (width 0.6) (layer "F.Cu") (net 4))
 (segment (start 233.528 113.424) (end 233.528 117.996) (width 0.6) (layer "F.Cu") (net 4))
 (segment (start 260.96 138.57) (end 260.96 114.948) (width 0.6) (layer "F.Cu") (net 4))
 (segment (start 234.036 121.552) (end 236.576 121.552) (width 0.6) (layer "F.Cu") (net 3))
 (segment (start 263.5 138.57) (end 263.5 114.44) (width 0.6) (layer "F.Cu") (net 3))
 (segment (start 259.944 110.884) (end 232.512 110.884) (width 0.6) (layer "F.Cu") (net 3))
 (segment (start 232.004 111.392) (end 232.004 119.52) (width 0.6) (layer "F.Cu") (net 3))
 (segment (start 232.004 119.52) (end 234.036 121.552) (width 0.6) (layer "F.Cu") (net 3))
 (segment (start 232.512 110.884) (end 232.004 111.392) (width 0.6) (layer "F.Cu") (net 3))
 (segment (start 263.5 114.44) (end 259.944 110.884) (width 0.6) (layer "F.Cu") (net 3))
 (segment (start 242.164 136.792) (end 239.116 136.792) (width 0.6) (layer "B.Cu") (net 32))
 (segment (start 268.58 118.25) (end 249.53 118.25) (width 0.6) (layer "B.Cu") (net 32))
 (segment (start 243.688 124.092) (end 243.688 135.268) (width 0.6) (layer "B.Cu") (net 32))
 (segment (start 243.688 135.268) (end 242.164 136.792) (width 0.6) (layer "B.Cu") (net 32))
 (segment (start 249.53 118.25) (end 243.688 124.092) (width 0.6) (layer "B.Cu") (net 32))
 (segment (start 242.672 129.172) (end 239.116 129.172) (width 0.6) (layer "F.Cu") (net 10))
 (segment (start 245.212 126.632) (end 242.672 129.172) (width 0.6) (layer "F.Cu") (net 10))
 (via (at 245.212 126.632) (size 0.9) (drill 0.6) (layers "F.Cu" "B.Cu") (free) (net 10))
 (segment (start 286.36 159.144) (end 286.36 144.412) (width 0.6) (layer "B.Cu") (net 10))
 (segment (start 246.228 127.14) (end 245.72 126.632) (width 0.6) (layer "B.Cu") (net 10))
 (segment (start 245.72 126.632) (end 245.212 126.632) (width 0.6) (layer "B.Cu") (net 10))
 (segment (start 285.344 143.396) (end 248.768 143.396) (width 0.6) (layer "B.Cu") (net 10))
 (segment (start 246.228 140.856) (end 246.228 127.14) (width 0.6) (layer "B.Cu") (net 10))
 (segment (start 286.36 144.412) (end 285.344 143.396) (width 0.6) (layer "B.Cu") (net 10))
 (segment (start 248.768 143.396) (end 246.228 140.856) (width 0.6) (layer "B.Cu") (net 10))
 (segment (start 242.164 157.62) (end 244.704 155.08) (width 0.6) (layer "F.Cu") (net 7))
 (segment (start 288.392 120.536) (end 290.17 118.758) (width 0.6) (layer "F.Cu") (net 7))
 (segment (start 244.704 155.08) (end 275.692 155.08) (width 0.6) (layer "F.Cu") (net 7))
 (segment (start 281.788 120.536) (end 288.392 120.536) (width 0.6) (layer "F.Cu") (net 7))
 (segment (start 290.17 118.758) (end 290.17 115.71) (width 0.6) (layer "F.Cu") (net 7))
 (segment (start 278.74 152.032) (end 278.74 123.584) (width 0.6) (layer "F.Cu") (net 7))
 (segment (start 278.74 123.584) (end 281.788 120.536) (width 0.6) (layer "F.Cu") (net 7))
 (segment (start 275.692 155.08) (end 278.74 152.032) (width 0.6) (layer "F.Cu") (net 7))
 (segment (start 239.116 162.192) (end 241.148 162.192) (width 0.6) (layer "F.Cu") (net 7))
 (segment (start 241.148 162.192) (end 242.164 161.176) (width 0.6) (layer "F.Cu") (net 7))
 (segment (start 242.164 161.176) (end 242.164 157.62) (width 0.6) (layer "F.Cu") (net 7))
 (segment (start 243.688 159.144) (end 246.228 156.604) (width 0.6) (layer "F.Cu") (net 8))
 (segment (start 241.148 164.732) (end 243.688 162.192) (width 0.6) (layer "F.Cu") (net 8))
 (segment (start 280.772 124.092) (end 282.804 122.06) (width 0.6) (layer "F.Cu") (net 8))
 (segment (start 282.804 122.06) (end 290.424 122.06) (width 0.6) (layer "F.Cu") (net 8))
 (segment (start 243.688 162.192) (end 243.688 159.144) (width 0.6) (layer "F.Cu") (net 8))
 (segment (start 279.248 156.604) (end 280.772 155.08) (width 0.6) (layer "F.Cu") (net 8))
 (segment (start 239.116 164.732) (end 241.148 164.732) (width 0.6) (layer "F.Cu") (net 8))
 (segment (start 246.228 156.604) (end 279.248 156.604) (width 0.6) (layer "F.Cu") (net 8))
 (segment (start 290.424 122.06) (end 292.71 119.774) (width 0.6) (layer "F.Cu") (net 8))
 (segment (start 292.71 119.774) (end 292.71 115.71) (width 0.6) (layer "F.Cu") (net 8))
 (segment (start 280.772 155.08) (end 280.772 124.092) (width 0.6) (layer "F.Cu") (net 8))
 (segment (start 283.82 126.632) (end 283.82 141.11) (width 0.6) (layer "F.Cu") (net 20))
 (segment (start 285.598 124.854) (end 283.82 126.632) (width 0.6) (layer "F.Cu") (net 20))
 (segment (start 298.678 124.854) (end 285.598 124.854) (width 0.6) (layer "F.Cu") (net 20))
 (segment (start 286.36 128.664) (end 286.36 141.11) (width 0.6) (layer "F.Cu") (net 21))
 (segment (start 287.63 127.394) (end 286.36 128.664) (width 0.6) (layer "F.Cu") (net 21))
 (segment (start 295.378 127.394) (end 287.63 127.394) (width 0.6) (layer "F.Cu") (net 21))
 (segment (start 290.17 129.934) (end 288.9 131.204) (width 0.6) (layer "F.Cu") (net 22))
 (segment (start 298.678 129.934) (end 290.17 129.934) (width 0.6) (layer "F.Cu") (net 22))
 (segment (start 288.9 131.204) (end 288.9 141.11) (width 0.6) (layer "F.Cu") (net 22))
 (segment (start 291.44 133.872) (end 292.838 132.474) (width 0.6) (layer "F.Cu") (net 23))
 (segment (start 291.44 141.11) (end 291.44 133.872) (width 0.6) (layer "F.Cu") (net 23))
 (segment (start 295.378 132.474) (end 292.838 132.474) (width 0.6) (layer "F.Cu") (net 23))
 (segment (start 234.544 191.148) (end 233.528 192.164) (width 0.6) (layer "F.Cu") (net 24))
 (segment (start 233.528 192.164) (end 233.528 193.7915) (width 0.6) (layer "F.Cu") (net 24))
 (segment (start 237.592 191.148) (end 234.544 191.148) (width 0.6) (layer "F.Cu") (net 24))
 (segment (start 286.36 167.272) (end 286.36 169.812) (width 0.6) (layer "F.Cu") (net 28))
 (segment (start 287.884 165.748) (end 286.36 167.272) (width 0.6) (layer "F.Cu") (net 28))
 (segment (start 233.528 197.244) (end 235.052 198.768) (width 0.6) (layer "F.Cu") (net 28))
 (segment (start 299.568 167.78) (end 297.536 165.748) (width 0.6) (layer "F.Cu") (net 28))
 (segment (start 235.052 198.768) (end 297.028 198.768) (width 0.6) (layer "F.Cu") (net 28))
 (segment (start 233.528 195.6165) (end 233.528 197.244) (width 0.6) (layer "F.Cu") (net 28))
 (segment (start 297.536 165.748) (end 287.884 165.748) (width 0.6) (layer "F.Cu") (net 28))
 (segment (start 297.028 198.768) (end 299.568 196.228) (width 0.6) (layer "F.Cu") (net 28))
 (segment (start 299.568 196.228) (end 299.568 167.78) (width 0.6) (layer "F.Cu") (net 28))
 (segment (start 237.592 193.688) (end 246.736 193.688) (width 0.6) (layer "F.Cu") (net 25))
 (segment (start 292.964 185.052) (end 292.964 183.02) (width 0.6) (layer "F.Cu") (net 25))
 (segment (start 287.376 177.94) (end 284.836 177.94) (width 0.6) (layer "F.Cu") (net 25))
 (segment (start 284.836 177.94) (end 251.816 177.94) (width 0.6) (layer "F.Cu") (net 25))
 (segment (start 250.292 190.132) (end 250.292 176.416) (width 0.6) (layer "F.Cu") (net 25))
 (segment (start 246.736 193.688) (end 250.292 190.132) (width 0.6) (layer "F.Cu") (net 25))
 (segment (start 288.9 169.812) (end 288.9 176.416) (width 0.6) (layer "F.Cu") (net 25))
 (segment (start 288.9 176.416) (end 287.376 177.94) (width 0.6) (layer "F.Cu") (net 25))
 (segment (start 287.884 177.94) (end 287.376 177.94) (width 0.6) (layer "F.Cu") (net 25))
 (segment (start 249.784 162.192) (end 247.244 162.192) (width 0.6) (layer "F.Cu") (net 25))
 (segment (start 292.964 183.02) (end 287.884 177.94) (width 0.6) (layer "F.Cu") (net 25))
 (segment (start 251.816 177.94) (end 250.292 176.416) (width 0.6) (layer "F.Cu") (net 25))
 (segment (start 250.292 162.7) (end 249.784 162.192) (width 0.6) (layer "F.Cu") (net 25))
 (segment (start 250.292 176.416) (end 250.292 162.7) (width 0.6) (layer "F.Cu") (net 25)))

